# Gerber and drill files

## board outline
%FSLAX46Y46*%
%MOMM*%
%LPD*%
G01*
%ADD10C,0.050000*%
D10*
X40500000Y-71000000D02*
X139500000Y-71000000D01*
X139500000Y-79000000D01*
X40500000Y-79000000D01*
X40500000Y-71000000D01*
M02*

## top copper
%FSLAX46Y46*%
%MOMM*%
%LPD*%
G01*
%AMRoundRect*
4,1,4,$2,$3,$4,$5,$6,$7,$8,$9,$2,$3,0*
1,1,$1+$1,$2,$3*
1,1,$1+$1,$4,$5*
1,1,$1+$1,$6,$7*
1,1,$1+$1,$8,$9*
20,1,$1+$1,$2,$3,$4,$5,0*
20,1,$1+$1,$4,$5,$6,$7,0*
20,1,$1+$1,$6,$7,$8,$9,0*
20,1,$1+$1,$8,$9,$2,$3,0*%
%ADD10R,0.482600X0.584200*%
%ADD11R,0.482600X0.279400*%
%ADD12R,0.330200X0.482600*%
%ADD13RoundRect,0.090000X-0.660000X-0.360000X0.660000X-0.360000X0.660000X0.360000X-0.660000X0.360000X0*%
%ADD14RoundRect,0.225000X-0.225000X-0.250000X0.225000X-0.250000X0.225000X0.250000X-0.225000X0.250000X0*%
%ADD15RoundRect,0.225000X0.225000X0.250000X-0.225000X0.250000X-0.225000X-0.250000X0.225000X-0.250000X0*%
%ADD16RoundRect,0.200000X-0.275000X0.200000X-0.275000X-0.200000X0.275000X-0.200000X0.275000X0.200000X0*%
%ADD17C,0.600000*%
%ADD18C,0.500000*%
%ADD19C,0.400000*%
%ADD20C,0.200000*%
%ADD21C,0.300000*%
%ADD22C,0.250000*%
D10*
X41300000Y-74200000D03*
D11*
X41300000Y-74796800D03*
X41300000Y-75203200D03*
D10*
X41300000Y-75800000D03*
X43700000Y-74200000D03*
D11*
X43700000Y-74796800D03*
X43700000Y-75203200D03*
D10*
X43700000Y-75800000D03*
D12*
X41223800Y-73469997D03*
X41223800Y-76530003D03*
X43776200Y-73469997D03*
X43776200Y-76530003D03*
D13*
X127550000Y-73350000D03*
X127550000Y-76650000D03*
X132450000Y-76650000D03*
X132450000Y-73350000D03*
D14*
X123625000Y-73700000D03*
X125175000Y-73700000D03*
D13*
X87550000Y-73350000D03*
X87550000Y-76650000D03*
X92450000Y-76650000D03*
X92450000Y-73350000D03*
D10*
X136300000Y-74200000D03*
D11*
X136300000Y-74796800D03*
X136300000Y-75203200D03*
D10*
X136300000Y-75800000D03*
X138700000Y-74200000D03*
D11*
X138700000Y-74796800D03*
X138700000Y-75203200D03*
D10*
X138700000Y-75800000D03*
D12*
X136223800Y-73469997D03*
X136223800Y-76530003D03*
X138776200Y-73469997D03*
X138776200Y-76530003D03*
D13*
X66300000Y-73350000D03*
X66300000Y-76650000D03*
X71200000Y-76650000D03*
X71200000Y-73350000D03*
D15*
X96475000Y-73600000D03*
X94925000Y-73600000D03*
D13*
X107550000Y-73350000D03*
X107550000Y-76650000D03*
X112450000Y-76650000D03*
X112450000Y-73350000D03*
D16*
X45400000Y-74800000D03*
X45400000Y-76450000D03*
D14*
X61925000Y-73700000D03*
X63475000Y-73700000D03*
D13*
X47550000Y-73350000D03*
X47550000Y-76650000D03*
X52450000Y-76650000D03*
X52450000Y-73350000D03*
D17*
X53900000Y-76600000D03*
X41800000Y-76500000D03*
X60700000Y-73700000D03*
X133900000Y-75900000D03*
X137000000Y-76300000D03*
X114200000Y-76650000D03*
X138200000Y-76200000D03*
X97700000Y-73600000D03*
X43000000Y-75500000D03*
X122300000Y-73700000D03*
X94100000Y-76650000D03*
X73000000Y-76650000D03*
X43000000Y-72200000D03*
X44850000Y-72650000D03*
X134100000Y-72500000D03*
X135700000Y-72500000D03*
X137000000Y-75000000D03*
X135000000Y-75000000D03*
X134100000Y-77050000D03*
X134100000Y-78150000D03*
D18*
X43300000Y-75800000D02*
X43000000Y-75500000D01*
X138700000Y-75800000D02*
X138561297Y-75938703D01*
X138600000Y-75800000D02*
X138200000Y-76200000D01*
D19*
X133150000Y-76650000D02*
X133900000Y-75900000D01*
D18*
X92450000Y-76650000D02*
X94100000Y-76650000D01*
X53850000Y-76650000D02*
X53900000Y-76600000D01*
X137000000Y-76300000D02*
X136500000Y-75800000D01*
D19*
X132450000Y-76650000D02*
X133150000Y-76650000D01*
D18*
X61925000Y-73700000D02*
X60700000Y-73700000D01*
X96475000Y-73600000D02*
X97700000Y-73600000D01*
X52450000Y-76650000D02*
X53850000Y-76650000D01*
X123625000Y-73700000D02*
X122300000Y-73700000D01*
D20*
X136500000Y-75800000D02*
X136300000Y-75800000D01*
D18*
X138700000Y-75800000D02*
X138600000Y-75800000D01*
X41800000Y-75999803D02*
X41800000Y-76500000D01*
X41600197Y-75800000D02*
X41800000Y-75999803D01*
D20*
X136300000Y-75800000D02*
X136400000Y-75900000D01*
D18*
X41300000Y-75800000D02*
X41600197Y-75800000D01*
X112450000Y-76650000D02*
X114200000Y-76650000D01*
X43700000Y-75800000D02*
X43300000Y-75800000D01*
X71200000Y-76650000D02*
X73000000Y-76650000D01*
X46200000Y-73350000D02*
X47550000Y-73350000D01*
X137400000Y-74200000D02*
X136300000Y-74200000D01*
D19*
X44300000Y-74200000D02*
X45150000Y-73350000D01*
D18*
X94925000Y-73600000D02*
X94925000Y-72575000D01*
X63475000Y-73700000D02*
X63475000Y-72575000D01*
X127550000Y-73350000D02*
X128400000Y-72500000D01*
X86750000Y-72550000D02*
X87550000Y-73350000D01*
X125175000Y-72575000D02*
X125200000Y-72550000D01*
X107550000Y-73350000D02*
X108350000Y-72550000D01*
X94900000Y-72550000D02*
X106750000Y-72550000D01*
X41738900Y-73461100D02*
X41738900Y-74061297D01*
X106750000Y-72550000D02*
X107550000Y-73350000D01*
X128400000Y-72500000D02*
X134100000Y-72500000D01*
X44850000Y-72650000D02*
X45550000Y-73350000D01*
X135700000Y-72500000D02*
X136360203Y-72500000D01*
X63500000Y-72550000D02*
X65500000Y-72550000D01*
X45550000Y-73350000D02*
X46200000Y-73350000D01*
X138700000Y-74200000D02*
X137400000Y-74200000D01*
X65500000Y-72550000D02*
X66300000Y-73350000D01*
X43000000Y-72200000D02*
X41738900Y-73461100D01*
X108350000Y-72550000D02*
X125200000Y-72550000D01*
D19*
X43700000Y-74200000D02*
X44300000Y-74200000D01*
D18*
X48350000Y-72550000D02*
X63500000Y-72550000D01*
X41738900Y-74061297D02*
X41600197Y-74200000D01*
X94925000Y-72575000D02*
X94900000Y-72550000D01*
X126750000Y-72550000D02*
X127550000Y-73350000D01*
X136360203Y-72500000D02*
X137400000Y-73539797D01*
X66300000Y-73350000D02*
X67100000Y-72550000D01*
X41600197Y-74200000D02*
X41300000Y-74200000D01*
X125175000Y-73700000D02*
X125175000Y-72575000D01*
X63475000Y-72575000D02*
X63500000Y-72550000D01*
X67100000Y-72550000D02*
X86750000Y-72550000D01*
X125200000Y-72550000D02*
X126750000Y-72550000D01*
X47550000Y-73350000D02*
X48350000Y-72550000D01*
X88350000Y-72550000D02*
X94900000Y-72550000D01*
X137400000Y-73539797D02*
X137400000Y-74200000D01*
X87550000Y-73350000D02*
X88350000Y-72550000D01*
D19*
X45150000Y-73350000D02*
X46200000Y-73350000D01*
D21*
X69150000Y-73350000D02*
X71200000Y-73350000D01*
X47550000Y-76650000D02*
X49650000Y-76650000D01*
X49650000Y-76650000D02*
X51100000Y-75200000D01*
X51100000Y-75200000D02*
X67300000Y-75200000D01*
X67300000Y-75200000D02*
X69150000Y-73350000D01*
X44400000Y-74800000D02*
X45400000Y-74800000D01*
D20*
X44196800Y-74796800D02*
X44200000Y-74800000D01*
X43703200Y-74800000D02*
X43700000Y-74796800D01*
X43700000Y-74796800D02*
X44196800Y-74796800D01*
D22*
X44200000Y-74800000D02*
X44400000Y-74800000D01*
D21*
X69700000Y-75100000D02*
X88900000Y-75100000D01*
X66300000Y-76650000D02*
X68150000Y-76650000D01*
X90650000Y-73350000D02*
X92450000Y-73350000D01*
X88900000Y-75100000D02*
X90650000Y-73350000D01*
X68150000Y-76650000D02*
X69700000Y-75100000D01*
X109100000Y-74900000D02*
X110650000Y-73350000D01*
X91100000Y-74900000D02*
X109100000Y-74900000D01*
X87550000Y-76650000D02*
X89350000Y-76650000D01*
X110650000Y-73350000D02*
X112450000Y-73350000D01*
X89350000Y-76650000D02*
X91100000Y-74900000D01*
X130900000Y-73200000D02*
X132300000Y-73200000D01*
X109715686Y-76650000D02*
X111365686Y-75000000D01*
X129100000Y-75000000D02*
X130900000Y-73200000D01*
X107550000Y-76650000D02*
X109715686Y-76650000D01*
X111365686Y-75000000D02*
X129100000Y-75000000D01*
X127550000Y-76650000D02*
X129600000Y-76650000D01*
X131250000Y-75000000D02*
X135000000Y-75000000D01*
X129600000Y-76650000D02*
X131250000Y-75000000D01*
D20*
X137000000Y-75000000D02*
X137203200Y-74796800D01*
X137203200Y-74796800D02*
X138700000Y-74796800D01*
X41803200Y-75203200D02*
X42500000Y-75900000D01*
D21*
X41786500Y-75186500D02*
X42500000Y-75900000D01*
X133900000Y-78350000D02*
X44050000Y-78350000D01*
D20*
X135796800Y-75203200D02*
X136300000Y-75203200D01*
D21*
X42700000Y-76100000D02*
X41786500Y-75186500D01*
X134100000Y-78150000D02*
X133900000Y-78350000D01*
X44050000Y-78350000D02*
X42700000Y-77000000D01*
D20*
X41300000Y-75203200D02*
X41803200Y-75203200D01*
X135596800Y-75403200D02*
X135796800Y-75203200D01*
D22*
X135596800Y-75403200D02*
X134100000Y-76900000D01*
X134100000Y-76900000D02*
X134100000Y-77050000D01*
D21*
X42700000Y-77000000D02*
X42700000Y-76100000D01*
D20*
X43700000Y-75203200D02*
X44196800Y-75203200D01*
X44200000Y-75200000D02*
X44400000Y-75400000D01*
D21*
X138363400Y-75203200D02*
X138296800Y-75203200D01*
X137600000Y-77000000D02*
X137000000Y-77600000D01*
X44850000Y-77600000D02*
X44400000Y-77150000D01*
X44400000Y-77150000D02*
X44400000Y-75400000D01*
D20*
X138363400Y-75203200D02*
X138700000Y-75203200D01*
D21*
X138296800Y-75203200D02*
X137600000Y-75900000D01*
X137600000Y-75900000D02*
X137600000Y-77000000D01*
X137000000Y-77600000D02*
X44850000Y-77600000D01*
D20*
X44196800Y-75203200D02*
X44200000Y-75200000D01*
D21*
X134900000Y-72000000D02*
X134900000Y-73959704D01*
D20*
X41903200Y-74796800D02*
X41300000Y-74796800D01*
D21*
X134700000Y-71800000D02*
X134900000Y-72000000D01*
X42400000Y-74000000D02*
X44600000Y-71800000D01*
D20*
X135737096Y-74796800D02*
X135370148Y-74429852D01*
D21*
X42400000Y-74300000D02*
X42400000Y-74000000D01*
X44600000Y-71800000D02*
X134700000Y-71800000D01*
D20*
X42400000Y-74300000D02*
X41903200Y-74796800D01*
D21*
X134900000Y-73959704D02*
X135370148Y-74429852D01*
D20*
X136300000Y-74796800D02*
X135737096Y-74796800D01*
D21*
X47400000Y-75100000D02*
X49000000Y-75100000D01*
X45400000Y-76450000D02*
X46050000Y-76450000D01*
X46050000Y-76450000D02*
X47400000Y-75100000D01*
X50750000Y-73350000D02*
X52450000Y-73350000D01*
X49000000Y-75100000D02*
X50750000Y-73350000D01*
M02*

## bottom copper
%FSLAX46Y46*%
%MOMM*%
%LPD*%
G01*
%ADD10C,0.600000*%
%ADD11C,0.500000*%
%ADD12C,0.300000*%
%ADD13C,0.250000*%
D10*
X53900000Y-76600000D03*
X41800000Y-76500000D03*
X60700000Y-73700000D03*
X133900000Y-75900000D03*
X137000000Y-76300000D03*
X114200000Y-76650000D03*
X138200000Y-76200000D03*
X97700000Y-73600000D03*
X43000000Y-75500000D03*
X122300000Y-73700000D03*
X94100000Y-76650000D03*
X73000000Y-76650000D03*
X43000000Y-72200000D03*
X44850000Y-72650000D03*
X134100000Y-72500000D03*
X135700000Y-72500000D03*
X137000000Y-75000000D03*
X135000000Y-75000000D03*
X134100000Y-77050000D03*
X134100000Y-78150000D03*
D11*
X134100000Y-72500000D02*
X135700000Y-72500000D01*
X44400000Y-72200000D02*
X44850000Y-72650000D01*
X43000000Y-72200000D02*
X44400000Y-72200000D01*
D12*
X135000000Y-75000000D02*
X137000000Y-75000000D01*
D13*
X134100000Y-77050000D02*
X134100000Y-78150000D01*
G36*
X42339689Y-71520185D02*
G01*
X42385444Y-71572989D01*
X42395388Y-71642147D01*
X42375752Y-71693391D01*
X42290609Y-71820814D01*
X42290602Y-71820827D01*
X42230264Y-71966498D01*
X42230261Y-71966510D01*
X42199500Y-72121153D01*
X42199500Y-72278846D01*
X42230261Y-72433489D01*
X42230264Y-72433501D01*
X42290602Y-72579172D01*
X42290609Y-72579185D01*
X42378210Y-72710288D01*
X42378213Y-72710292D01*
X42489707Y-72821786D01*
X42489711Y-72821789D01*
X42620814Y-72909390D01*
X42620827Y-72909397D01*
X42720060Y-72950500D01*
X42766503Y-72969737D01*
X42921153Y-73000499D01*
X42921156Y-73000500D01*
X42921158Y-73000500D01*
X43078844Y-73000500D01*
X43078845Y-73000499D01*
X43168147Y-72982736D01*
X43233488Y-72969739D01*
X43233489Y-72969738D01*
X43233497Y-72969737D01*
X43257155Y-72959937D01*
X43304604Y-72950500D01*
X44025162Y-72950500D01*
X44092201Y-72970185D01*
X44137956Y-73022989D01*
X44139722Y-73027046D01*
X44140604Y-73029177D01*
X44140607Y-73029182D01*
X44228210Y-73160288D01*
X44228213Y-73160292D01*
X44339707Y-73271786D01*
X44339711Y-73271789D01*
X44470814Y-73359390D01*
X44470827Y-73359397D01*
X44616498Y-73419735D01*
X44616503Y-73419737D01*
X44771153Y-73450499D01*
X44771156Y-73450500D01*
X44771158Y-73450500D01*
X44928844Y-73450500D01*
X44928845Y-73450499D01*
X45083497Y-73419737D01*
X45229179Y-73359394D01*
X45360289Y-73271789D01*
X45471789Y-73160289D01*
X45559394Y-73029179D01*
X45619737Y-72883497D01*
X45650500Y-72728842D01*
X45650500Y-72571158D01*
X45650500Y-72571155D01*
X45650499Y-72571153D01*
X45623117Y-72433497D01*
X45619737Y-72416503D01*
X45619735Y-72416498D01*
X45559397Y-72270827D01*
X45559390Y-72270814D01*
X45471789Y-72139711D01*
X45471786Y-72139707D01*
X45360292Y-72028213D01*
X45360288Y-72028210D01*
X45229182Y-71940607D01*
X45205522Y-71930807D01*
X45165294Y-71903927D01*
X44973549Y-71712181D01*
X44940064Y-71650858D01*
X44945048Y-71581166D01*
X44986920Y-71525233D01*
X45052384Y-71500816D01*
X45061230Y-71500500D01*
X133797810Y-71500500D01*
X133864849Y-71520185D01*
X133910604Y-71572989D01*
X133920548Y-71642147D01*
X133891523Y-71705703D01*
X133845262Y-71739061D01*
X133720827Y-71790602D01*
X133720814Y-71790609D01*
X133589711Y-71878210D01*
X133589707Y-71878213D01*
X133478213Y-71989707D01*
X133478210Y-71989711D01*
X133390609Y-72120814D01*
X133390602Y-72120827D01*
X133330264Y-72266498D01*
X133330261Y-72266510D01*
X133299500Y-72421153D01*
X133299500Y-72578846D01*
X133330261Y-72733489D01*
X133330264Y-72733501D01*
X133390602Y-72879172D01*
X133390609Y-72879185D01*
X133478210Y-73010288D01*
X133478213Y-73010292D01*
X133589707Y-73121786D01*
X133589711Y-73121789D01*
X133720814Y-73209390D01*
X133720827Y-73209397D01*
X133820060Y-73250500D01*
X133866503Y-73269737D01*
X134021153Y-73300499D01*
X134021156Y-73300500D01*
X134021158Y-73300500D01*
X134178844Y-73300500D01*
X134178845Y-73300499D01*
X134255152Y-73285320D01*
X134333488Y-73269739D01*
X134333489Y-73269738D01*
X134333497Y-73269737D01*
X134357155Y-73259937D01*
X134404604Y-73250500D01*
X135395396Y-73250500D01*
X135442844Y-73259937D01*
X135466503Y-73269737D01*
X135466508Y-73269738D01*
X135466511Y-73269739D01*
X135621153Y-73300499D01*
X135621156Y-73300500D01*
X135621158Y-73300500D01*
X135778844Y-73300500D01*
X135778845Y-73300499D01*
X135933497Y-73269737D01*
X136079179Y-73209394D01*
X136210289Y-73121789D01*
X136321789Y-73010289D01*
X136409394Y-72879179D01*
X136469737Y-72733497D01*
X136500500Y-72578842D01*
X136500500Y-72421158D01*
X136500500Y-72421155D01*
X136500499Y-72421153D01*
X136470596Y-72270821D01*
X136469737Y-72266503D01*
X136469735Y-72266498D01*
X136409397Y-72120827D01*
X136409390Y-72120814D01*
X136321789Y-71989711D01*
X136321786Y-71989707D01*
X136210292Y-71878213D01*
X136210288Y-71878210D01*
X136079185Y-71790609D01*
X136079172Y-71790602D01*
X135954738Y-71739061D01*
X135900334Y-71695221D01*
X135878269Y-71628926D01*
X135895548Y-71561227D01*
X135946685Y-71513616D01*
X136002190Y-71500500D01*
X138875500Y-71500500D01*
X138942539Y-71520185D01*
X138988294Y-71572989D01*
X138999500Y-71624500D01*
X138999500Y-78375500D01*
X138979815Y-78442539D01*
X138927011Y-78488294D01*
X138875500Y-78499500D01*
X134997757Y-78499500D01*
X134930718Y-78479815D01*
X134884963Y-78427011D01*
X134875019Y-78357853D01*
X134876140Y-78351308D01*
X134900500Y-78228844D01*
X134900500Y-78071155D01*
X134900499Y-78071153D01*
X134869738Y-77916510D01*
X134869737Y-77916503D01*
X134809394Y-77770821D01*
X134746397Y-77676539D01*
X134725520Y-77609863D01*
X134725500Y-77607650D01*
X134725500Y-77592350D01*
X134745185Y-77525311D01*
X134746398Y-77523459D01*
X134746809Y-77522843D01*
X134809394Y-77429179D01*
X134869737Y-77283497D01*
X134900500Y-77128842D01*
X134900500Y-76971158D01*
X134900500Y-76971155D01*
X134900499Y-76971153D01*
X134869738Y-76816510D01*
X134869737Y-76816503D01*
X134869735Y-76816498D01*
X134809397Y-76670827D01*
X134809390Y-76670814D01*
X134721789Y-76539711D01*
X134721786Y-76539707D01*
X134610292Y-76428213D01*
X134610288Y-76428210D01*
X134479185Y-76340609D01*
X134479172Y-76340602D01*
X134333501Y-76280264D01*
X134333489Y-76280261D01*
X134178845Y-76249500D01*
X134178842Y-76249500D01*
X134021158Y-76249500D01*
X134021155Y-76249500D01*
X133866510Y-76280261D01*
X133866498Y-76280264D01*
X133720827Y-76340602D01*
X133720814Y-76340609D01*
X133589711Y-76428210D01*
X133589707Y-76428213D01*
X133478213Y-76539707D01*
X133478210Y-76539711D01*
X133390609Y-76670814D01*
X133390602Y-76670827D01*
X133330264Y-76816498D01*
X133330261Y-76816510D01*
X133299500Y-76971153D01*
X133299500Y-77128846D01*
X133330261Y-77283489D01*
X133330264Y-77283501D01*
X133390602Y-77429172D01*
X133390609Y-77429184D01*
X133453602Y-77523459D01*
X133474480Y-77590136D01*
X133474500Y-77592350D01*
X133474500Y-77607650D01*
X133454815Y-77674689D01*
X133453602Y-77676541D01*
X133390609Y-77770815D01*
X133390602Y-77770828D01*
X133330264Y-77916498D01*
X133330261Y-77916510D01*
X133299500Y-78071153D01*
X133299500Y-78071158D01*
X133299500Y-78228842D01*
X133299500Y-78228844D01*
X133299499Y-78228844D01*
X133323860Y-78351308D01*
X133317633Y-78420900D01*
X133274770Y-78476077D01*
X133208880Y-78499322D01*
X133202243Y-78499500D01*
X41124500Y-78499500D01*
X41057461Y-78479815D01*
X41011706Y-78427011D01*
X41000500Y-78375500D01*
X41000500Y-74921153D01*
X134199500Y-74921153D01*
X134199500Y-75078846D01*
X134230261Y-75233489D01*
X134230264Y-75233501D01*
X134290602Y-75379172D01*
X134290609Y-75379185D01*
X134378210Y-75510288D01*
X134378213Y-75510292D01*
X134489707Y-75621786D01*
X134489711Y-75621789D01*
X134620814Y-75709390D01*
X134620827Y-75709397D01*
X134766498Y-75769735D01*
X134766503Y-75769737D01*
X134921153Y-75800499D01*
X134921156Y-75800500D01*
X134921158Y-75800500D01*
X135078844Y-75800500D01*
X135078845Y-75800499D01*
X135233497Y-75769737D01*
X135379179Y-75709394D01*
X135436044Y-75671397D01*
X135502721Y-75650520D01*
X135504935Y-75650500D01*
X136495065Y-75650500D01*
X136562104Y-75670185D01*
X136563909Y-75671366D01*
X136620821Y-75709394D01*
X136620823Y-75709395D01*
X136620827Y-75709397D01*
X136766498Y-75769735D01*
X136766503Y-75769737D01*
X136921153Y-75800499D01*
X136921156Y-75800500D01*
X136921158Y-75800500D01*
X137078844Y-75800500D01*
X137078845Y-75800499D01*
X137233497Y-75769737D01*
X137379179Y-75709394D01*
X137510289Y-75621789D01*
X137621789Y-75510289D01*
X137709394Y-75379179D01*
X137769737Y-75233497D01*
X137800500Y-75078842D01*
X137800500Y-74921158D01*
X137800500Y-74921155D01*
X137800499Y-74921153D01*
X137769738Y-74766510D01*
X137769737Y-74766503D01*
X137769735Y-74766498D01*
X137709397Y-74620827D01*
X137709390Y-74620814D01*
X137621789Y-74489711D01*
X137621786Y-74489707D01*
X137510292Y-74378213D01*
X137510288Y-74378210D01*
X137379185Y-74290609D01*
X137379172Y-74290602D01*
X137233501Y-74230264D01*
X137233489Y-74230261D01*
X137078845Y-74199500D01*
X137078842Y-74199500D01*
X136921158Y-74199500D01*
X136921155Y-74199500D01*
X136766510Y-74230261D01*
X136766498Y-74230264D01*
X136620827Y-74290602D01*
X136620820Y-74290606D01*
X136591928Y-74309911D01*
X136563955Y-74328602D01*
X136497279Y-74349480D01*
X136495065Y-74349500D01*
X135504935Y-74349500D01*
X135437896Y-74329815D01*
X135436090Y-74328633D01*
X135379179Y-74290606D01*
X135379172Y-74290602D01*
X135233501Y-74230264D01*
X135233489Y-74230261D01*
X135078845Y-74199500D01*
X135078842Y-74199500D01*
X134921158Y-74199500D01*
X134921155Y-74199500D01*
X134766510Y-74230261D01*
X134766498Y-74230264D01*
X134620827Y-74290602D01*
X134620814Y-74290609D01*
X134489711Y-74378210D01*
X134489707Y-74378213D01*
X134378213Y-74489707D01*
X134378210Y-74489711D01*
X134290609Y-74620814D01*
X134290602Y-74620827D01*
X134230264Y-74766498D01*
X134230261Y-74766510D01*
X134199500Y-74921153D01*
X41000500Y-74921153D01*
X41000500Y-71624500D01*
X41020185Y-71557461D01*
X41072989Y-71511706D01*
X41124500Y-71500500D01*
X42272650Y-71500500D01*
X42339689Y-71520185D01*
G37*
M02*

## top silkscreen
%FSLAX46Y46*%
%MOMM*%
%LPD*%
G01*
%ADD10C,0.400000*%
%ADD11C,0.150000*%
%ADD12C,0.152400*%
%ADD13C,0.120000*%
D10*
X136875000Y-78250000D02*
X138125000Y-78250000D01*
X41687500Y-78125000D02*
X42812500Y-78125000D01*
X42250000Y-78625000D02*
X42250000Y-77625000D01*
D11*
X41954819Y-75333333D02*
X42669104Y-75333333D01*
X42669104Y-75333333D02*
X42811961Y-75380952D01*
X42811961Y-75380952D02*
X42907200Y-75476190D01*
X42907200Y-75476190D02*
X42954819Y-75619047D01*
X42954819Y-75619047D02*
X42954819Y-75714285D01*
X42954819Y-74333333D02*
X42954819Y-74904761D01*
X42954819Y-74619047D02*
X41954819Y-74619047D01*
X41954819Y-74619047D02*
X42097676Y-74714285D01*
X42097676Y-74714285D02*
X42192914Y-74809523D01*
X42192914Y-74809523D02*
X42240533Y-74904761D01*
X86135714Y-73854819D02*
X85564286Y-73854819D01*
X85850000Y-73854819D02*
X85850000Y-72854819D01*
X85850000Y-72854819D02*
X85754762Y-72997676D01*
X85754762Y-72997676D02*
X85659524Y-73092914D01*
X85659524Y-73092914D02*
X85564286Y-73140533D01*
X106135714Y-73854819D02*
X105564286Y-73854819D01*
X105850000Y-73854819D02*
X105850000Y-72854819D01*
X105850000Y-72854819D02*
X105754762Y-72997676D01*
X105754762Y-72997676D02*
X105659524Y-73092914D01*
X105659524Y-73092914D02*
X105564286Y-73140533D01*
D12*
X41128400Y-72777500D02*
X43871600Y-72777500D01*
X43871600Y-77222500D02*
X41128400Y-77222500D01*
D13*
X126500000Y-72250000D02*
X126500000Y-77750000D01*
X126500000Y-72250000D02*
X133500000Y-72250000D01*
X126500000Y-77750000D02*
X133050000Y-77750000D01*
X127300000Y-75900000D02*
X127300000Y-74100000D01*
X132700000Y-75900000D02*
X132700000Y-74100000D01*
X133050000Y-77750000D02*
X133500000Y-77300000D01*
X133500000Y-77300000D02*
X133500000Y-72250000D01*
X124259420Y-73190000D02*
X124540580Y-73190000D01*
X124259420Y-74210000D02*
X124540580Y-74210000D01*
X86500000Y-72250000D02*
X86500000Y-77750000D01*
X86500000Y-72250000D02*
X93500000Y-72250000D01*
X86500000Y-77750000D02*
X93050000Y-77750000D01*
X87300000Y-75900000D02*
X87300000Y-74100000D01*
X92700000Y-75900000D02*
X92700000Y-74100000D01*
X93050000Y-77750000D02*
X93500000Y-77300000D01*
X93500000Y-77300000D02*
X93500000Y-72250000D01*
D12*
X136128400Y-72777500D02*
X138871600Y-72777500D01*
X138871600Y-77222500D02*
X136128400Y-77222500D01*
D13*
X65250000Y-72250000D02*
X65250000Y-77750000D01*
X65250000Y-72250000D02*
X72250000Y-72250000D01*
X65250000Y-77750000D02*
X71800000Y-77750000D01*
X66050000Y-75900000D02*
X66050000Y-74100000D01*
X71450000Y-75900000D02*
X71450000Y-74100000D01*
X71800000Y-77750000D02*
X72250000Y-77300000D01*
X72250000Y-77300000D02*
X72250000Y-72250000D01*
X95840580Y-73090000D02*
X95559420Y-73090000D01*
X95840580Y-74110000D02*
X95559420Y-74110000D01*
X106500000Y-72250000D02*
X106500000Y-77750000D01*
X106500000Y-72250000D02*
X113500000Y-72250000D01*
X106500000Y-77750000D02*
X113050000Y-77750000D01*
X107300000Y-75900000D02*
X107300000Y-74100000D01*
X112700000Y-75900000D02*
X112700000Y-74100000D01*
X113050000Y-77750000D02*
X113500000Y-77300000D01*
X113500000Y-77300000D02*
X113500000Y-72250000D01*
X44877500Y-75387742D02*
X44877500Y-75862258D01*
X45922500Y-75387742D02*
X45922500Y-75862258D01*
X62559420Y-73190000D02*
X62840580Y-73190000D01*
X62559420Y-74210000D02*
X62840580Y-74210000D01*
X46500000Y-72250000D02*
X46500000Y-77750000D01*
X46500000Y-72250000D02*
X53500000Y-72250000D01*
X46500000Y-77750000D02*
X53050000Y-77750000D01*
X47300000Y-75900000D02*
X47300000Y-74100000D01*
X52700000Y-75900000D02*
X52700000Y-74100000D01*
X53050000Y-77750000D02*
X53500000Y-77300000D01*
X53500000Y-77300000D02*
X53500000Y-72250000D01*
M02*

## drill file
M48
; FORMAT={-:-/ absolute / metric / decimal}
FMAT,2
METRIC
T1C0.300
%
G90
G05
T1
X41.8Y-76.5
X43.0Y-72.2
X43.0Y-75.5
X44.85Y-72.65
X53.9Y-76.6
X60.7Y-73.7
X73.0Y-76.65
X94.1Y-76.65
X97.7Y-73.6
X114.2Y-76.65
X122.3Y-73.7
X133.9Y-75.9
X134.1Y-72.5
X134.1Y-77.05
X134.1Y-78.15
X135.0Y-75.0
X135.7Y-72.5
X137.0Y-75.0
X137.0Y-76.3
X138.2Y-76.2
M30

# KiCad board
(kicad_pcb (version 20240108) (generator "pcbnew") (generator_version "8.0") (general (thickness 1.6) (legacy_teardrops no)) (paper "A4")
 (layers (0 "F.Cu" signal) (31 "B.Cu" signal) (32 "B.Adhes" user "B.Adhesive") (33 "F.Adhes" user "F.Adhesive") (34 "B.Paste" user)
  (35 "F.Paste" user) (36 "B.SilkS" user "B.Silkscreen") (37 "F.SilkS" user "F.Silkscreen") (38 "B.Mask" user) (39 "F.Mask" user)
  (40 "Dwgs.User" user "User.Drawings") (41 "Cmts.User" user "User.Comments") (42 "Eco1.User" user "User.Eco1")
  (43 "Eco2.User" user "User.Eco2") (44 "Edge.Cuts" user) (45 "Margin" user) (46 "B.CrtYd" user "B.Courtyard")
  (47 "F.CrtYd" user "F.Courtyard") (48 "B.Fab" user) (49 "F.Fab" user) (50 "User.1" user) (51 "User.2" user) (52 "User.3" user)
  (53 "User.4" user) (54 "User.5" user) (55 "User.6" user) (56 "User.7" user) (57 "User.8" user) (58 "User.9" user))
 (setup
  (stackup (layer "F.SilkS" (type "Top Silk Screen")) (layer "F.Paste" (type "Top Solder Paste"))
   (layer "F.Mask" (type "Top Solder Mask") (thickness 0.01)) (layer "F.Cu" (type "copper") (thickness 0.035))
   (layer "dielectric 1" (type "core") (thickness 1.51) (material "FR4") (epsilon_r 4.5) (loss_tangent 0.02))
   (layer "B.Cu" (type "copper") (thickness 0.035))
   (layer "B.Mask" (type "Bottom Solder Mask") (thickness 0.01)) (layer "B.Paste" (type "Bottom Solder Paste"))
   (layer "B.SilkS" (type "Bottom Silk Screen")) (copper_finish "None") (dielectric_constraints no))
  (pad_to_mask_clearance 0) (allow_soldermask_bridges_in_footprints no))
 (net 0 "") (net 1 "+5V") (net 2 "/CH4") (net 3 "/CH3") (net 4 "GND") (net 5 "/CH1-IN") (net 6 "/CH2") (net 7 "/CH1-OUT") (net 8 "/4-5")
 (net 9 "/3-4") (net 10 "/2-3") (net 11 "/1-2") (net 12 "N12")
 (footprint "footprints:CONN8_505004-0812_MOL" (layer "F.Cu") (at 42.5 75 90)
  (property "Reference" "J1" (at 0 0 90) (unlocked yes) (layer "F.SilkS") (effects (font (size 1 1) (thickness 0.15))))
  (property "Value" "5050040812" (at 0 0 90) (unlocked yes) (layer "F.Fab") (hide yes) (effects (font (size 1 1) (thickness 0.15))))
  (fp_line (start 2.2225 -1.3716) (end 2.2225 1.3716) (stroke (width 0.1524) (type solid)) (layer "F.SilkS"))
  (fp_line (start -2.2225 1.3716) (end -2.2225 -1.3716) (stroke (width 0.1524) (type solid)) (layer "F.SilkS"))
  (pad "1" smd rect (at 0.8 -1.2 90) (size 0.5842 0.4826) (layers "F.Cu" "F.Paste" "F.Mask") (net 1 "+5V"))
  (pad "2" smd rect (at 0.2032 -1.2 90) (size 0.2794 0.4826) (layers "F.Cu" "F.Paste" "F.Mask") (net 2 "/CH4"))
  (pad "3" smd rect (at -0.2032 -1.2 90) (size 0.2794 0.4826) (layers "F.Cu" "F.Paste" "F.Mask") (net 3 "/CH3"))
  (pad "4" smd rect (at -0.8 -1.2 90) (size 0.5842 0.4826) (layers "F.Cu" "F.Paste" "F.Mask") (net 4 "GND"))
  (pad "5" smd rect (at 0.8 1.2 90) (size 0.5842 0.4826) (layers "F.Cu" "F.Paste" "F.Mask") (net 1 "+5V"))
  (pad "6" smd rect (at 0.2032 1.2 90) (size 0.2794 0.4826) (layers "F.Cu" "F.Paste" "F.Mask") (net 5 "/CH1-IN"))
  (pad "7" smd rect (at -0.2032 1.2 90) (size 0.2794 0.4826) (layers "F.Cu" "F.Paste" "F.Mask") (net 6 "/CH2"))
  (pad "8" smd rect (at -0.8 1.2 90) (size 0.5842 0.4826) (layers "F.Cu" "F.Paste" "F.Mask") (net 4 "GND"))
  (pad "9" smd rect (at 1.530003 -1.2762 90) (size 0.4826 0.3302) (layers "F.Cu" "F.Paste" "F.Mask"))
  (pad "10" smd rect (at -1.530003 -1.2762 90) (size 0.4826 0.3302) (layers "F.Cu" "F.Paste" "F.Mask"))
  (pad "11" smd rect (at 1.530003 1.2762 90) (size 0.4826 0.3302) (layers "F.Cu" "F.Paste" "F.Mask"))
  (pad "12" smd rect (at -1.530003 1.2762 90) (size 0.4826 0.3302) (layers "F.Cu" "F.Paste" "F.Mask")))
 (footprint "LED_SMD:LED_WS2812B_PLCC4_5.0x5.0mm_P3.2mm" (layer "F.Cu") (at 130 75)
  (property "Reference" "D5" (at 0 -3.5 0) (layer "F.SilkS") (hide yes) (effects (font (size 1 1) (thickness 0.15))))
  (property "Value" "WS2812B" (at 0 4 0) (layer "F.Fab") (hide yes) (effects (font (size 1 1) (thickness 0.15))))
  (fp_line (start -3.5 -2.75) (end -3.5 2.75) (stroke (width 0.12) (type default)) (layer "F.SilkS"))
  (fp_line (start -3.5 -2.75) (end 3.5 -2.75) (stroke (width 0.12) (type solid)) (layer "F.SilkS"))
  (fp_line (start -3.5 2.75) (end 3.05 2.75) (stroke (width 0.12) (type solid)) (layer "F.SilkS"))
  (fp_line (start -2.7 0.9) (end -2.7 -0.9) (stroke (width 0.12) (type default)) (layer "F.SilkS"))
  (fp_line (start 2.7 0.9) (end 2.7 -0.9) (stroke (width 0.12) (type default)) (layer "F.SilkS"))
  (fp_line (start 3.05 2.75) (end 3.5 2.3) (stroke (width 0.12) (type default)) (layer "F.SilkS"))
  (fp_line (start 3.5 2.3) (end 3.5 -2.75) (stroke (width 0.12) (type default)) (layer "F.SilkS"))
  (pad "1" smd roundrect (at -2.45 -1.65) (size 1.5 0.9) (layers "F.Cu" "F.Paste" "F.Mask") (roundrect_rratio 0.1) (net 1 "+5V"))
  (pad "2" smd roundrect (at -2.45 1.65) (size 1.5 0.9) (layers "F.Cu" "F.Paste" "F.Mask") (roundrect_rratio 0.1) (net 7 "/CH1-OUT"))
  (pad "3" smd roundrect (at 2.45 1.65) (size 1.5 0.9) (layers "F.Cu" "F.Paste" "F.Mask") (roundrect_rratio 0.1) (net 4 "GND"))
  (pad "4" smd roundrect (at 2.45 -1.65) (size 1.5 0.9) (layers "F.Cu" "F.Paste" "F.Mask") (roundrect_rratio 0.1) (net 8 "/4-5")))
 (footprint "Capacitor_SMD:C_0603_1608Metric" (layer "F.Cu") (at 124.4 73.7)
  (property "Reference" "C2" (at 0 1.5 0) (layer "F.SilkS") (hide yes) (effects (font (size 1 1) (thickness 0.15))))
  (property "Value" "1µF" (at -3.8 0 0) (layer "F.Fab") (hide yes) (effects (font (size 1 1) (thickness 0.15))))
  (fp_line (start -0.14058 -0.51) (end 0.14058 -0.51) (stroke (width 0.12) (type solid)) (layer "F.SilkS"))
  (fp_line (start -0.14058 0.51) (end 0.14058 0.51) (stroke (width 0.12) (type solid)) (layer "F.SilkS"))
  (pad "1" smd roundrect (at -0.775 0) (size 0.9 0.95) (layers "F.Cu" "F.Paste" "F.Mask") (roundrect_rratio 0.25) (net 4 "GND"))
  (pad "2" smd roundrect (at 0.775 0) (size 0.9 0.95) (layers "F.Cu" "F.Paste" "F.Mask") (roundrect_rratio 0.25) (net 1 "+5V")))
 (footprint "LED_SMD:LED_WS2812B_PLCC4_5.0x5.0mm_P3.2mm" (layer "F.Cu") (at 90 75)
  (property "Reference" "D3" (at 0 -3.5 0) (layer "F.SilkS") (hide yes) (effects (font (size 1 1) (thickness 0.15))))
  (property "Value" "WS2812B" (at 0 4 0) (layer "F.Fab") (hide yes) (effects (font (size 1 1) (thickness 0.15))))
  (fp_line (start -3.5 -2.75) (end -3.5 2.75) (stroke (width 0.12) (type default)) (layer "F.SilkS"))
  (fp_line (start -3.5 -2.75) (end 3.5 -2.75) (stroke (width 0.12) (type solid)) (layer "F.SilkS"))
  (fp_line (start -3.5 2.75) (end 3.05 2.75) (stroke (width 0.12) (type solid)) (layer "F.SilkS"))
  (fp_line (start -2.7 0.9) (end -2.7 -0.9) (stroke (width 0.12) (type default)) (layer "F.SilkS"))
  (fp_line (start 2.7 0.9) (end 2.7 -0.9) (stroke (width 0.12) (type default)) (layer "F.SilkS"))
  (fp_line (start 3.05 2.75) (end 3.5 2.3) (stroke (width 0.12) (type default)) (layer "F.SilkS"))
  (fp_line (start 3.5 2.3) (end 3.5 -2.75) (stroke (width 0.12) (type default)) (layer "F.SilkS"))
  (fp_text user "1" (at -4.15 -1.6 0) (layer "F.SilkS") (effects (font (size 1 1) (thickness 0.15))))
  (pad "1" smd roundrect (at -2.45 -1.65) (size 1.5 0.9) (layers "F.Cu" "F.Paste" "F.Mask") (roundrect_rratio 0.1) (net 1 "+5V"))
  (pad "2" smd roundrect (at -2.45 1.65) (size 1.5 0.9) (layers "F.Cu" "F.Paste" "F.Mask") (roundrect_rratio 0.1) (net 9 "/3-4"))
  (pad "3" smd roundrect (at 2.45 1.65) (size 1.5 0.9) (layers "F.Cu" "F.Paste" "F.Mask") (roundrect_rratio 0.1) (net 4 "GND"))
  (pad "4" smd roundrect (at 2.45 -1.65) (size 1.5 0.9) (layers "F.Cu" "F.Paste" "F.Mask") (roundrect_rratio 0.1) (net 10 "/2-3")))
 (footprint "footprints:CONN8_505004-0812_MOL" (layer "F.Cu") (at 137.5 75 90)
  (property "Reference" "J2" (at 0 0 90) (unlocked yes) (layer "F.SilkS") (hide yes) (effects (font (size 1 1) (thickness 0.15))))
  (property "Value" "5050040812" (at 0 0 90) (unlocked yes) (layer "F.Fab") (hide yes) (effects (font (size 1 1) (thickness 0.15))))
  (fp_line (start 2.2225 -1.3716) (end 2.2225 1.3716) (stroke (width 0.1524) (type solid)) (layer "F.SilkS"))
  (fp_line (start -2.2225 1.3716) (end -2.2225 -1.3716) (stroke (width 0.1524) (type solid)) (layer "F.SilkS"))
  (pad "1" smd rect (at 0.8 -1.2 90) (size 0.5842 0.4826) (layers "F.Cu" "F.Paste" "F.Mask") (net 1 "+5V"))
  (pad "2" smd rect (at 0.2032 -1.2 90) (size 0.2794 0.4826) (layers "F.Cu" "F.Paste" "F.Mask") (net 2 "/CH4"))
  (pad "3" smd rect (at -0.2032 -1.2 90) (size 0.2794 0.4826) (layers "F.Cu" "F.Paste" "F.Mask") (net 3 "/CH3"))
  (pad "4" smd rect (at -0.8 -1.2 90) (size 0.5842 0.4826) (layers "F.Cu" "F.Paste" "F.Mask") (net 4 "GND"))
  (pad "5" smd rect (at 0.8 1.2 90) (size 0.5842 0.4826) (layers "F.Cu" "F.Paste" "F.Mask") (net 1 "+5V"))
  (pad "6" smd rect (at 0.2032 1.2 90) (size 0.2794 0.4826) (layers "F.Cu" "F.Paste" "F.Mask") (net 7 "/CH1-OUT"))
  (pad "7" smd rect (at -0.2032 1.2 90) (size 0.2794 0.4826) (layers "F.Cu" "F.Paste" "F.Mask") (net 6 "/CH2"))
  (pad "8" smd rect (at -0.8 1.2 90) (size 0.5842 0.4826) (layers "F.Cu" "F.Paste" "F.Mask") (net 4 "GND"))
  (pad "9" smd rect (at 1.530003 -1.2762 90) (size 0.4826 0.3302) (layers "F.Cu" "F.Paste" "F.Mask"))
  (pad "10" smd rect (at -1.530003 -1.2762 90) (size 0.4826 0.3302) (layers "F.Cu" "F.Paste" "F.Mask"))
  (pad "11" smd rect (at 1.530003 1.2762 90) (size 0.4826 0.3302) (layers "F.Cu" "F.Paste" "F.Mask"))
  (pad "12" smd rect (at -1.530003 1.2762 90) (size 0.4826 0.3302) (layers "F.Cu" "F.Paste" "F.Mask")))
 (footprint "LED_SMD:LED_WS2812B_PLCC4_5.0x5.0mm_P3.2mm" (layer "F.Cu") (at 68.75 75)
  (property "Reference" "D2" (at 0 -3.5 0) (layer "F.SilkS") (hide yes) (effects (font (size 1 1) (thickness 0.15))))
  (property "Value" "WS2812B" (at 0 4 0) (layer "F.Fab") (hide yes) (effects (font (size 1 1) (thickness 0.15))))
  (fp_line (start -3.5 -2.75) (end -3.5 2.75) (stroke (width 0.12) (type default)) (layer "F.SilkS"))
  (fp_line (start -3.5 -2.75) (end 3.5 -2.75) (stroke (width 0.12) (type solid)) (layer "F.SilkS"))
  (fp_line (start -3.5 2.75) (end 3.05 2.75) (stroke (width 0.12) (type solid)) (layer "F.SilkS"))
  (fp_line (start -2.7 0.9) (end -2.7 -0.9) (stroke (width 0.12) (type default)) (layer "F.SilkS"))
  (fp_line (start 2.7 0.9) (end 2.7 -0.9) (stroke (width 0.12) (type default)) (layer "F.SilkS"))
  (fp_line (start 3.05 2.75) (end 3.5 2.3) (stroke (width 0.12) (type default)) (layer "F.SilkS"))
  (fp_line (start 3.5 2.3) (end 3.5 -2.75) (stroke (width 0.12) (type default)) (layer "F.SilkS"))
  (pad "1" smd roundrect (at -2.45 -1.65) (size 1.5 0.9) (layers "F.Cu" "F.Paste" "F.Mask") (roundrect_rratio 0.1) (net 1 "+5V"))
  (pad "2" smd roundrect (at -2.45 1.65) (size 1.5 0.9) (layers "F.Cu" "F.Paste" "F.Mask") (roundrect_rratio 0.1) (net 10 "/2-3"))
  (pad "3" smd roundrect (at 2.45 1.65) (size 1.5 0.9) (layers "F.Cu" "F.Paste" "F.Mask") (roundrect_rratio 0.1) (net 4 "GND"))
  (pad "4" smd roundrect (at 2.45 -1.65) (size 1.5 0.9) (layers "F.Cu" "F.Paste" "F.Mask") (roundrect_rratio 0.1) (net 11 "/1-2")))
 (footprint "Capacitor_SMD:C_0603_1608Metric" (layer "F.Cu") (at 95.7 73.6 180)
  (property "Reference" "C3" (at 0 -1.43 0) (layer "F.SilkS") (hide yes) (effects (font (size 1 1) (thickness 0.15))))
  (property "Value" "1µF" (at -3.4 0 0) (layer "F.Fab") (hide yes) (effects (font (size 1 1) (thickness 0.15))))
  (fp_line (start -0.14058 0.51) (end 0.14058 0.51) (stroke (width 0.12) (type solid)) (layer "F.SilkS"))
  (fp_line (start -0.14058 -0.51) (end 0.14058 -0.51) (stroke (width 0.12) (type solid)) (layer "F.SilkS"))
  (pad "1" smd roundrect (at -0.775 0 180) (size 0.9 0.95) (layers "F.Cu" "F.Paste" "F.Mask") (roundrect_rratio 0.25) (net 4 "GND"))
  (pad "2" smd roundrect (at 0.775 0 180) (size 0.9 0.95) (layers "F.Cu" "F.Paste" "F.Mask") (roundrect_rratio 0.25) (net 1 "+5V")))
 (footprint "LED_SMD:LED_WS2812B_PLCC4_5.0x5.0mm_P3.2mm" (layer "F.Cu") (at 110 75)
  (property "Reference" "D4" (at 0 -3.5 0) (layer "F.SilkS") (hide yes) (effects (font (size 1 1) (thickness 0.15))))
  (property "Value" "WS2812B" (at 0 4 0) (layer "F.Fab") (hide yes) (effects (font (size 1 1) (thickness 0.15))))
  (fp_line (start -3.5 -2.75) (end -3.5 2.75) (stroke (width 0.12) (type default)) (layer "F.SilkS"))
  (fp_line (start -3.5 -2.75) (end 3.5 -2.75) (stroke (width 0.12) (type solid)) (layer "F.SilkS"))
  (fp_line (start -3.5 2.75) (end 3.05 2.75) (stroke (width 0.12) (type solid)) (layer "F.SilkS"))
  (fp_line (start -2.7 0.9) (end -2.7 -0.9) (stroke (width 0.12) (type default)) (layer "F.SilkS"))
  (fp_line (start 2.7 0.9) (end 2.7 -0.9) (stroke (width 0.12) (type default)) (layer "F.SilkS"))
  (fp_line (start 3.05 2.75) (end 3.5 2.3) (stroke (width 0.12) (type default)) (layer "F.SilkS"))
  (fp_line (start 3.5 2.3) (end 3.5 -2.75) (stroke (width 0.12) (type default)) (layer "F.SilkS"))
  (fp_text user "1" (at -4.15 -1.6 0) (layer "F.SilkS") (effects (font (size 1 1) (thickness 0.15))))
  (pad "1" smd roundrect (at -2.45 -1.65) (size 1.5 0.9) (layers "F.Cu" "F.Paste" "F.Mask") (roundrect_rratio 0.1) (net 1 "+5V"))
  (pad "2" smd roundrect (at -2.45 1.65) (size 1.5 0.9) (layers "F.Cu" "F.Paste" "F.Mask") (roundrect_rratio 0.1) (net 8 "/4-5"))
  (pad "3" smd roundrect (at 2.45 1.65) (size 1.5 0.9) (layers "F.Cu" "F.Paste" "F.Mask") (roundrect_rratio 0.1) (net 4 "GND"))
  (pad "4" smd roundrect (at 2.45 -1.65) (size 1.5 0.9) (layers "F.Cu" "F.Paste" "F.Mask") (roundrect_rratio 0.1) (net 9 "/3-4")))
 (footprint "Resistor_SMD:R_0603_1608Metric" (layer "F.Cu") (at 45.4 75.625 -90)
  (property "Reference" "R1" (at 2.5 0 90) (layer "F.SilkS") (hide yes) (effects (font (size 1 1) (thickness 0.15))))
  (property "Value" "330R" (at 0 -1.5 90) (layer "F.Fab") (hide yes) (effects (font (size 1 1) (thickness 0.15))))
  (fp_line (start -0.237258 0.5225) (end 0.237258 0.5225) (stroke (width 0.12) (type solid)) (layer "F.SilkS"))
  (fp_line (start -0.237258 -0.5225) (end 0.237258 -0.5225) (stroke (width 0.12) (type solid)) (layer "F.SilkS"))
  (pad "1" smd roundrect (at -0.825 0 270) (size 0.8 0.95) (layers "F.Cu" "F.Paste" "F.Mask") (roundrect_rratio 0.25) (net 5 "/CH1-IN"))
  (pad "2" smd roundrect (at 0.825 0 270) (size 0.8 0.95) (layers "F.Cu" "F.Paste" "F.Mask") (roundrect_rratio 0.25) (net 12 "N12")))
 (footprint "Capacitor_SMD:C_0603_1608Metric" (layer "F.Cu") (at 62.7 73.7)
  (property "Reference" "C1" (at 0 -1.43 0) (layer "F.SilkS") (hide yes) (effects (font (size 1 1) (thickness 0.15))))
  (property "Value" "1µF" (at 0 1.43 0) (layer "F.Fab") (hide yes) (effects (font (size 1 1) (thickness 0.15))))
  (fp_line (start -0.14058 -0.51) (end 0.14058 -0.51) (stroke (width 0.12) (type solid)) (layer "F.SilkS"))
  (fp_line (start -0.14058 0.51) (end 0.14058 0.51) (stroke (width 0.12) (type solid)) (layer "F.SilkS"))
  (pad "1" smd roundrect (at -0.775 0) (size 0.9 0.95) (layers "F.Cu" "F.Paste" "F.Mask") (roundrect_rratio 0.25) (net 4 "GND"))
  (pad "2" smd roundrect (at 0.775 0) (size 0.9 0.95) (layers "F.Cu" "F.Paste" "F.Mask") (roundrect_rratio 0.25) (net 1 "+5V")))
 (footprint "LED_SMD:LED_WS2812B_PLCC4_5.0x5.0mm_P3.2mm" (layer "F.Cu") (at 50 75)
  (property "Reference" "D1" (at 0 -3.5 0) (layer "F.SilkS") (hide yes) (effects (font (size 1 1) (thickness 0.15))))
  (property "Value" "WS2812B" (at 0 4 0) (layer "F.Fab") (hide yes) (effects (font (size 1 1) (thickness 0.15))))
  (fp_line (start -3.5 -2.75) (end -3.5 2.75) (stroke (width 0.12) (type default)) (layer "F.SilkS"))
  (fp_line (start -3.5 -2.75) (end 3.5 -2.75) (stroke (width 0.12) (type solid)) (layer "F.SilkS"))
  (fp_line (start -3.5 2.75) (end 3.05 2.75) (stroke (width 0.12) (type solid)) (layer "F.SilkS"))
  (fp_line (start -2.7 0.9) (end -2.7 -0.9) (stroke (width 0.12) (type default)) (layer "F.SilkS"))
  (fp_line (start 2.7 0.9) (end 2.7 -0.9) (stroke (width 0.12) (type default)) (layer "F.SilkS"))
  (fp_line (start 3.05 2.75) (end 3.5 2.3) (stroke (width 0.12) (type default)) (layer "F.SilkS"))
  (fp_line (start 3.5 2.3) (end 3.5 -2.75) (stroke (width 0.12) (type default)) (layer "F.SilkS"))
  (pad "1" smd roundrect (at -2.45 -1.65) (size 1.5 0.9) (layers "F.Cu" "F.Paste" "F.Mask") (roundrect_rratio 0.1) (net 1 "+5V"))
  (pad "2" smd roundrect (at -2.45 1.65) (size 1.5 0.9) (layers "F.Cu" "F.Paste" "F.Mask") (roundrect_rratio 0.1) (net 11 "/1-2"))
  (pad "3" smd roundrect (at 2.45 1.65) (size 1.5 0.9) (layers "F.Cu" "F.Paste" "F.Mask") (roundrect_rratio 0.1) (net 4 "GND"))
  (pad "4" smd roundrect (at 2.45 -1.65) (size 1.5 0.9) (layers "F.Cu" "F.Paste" "F.Mask") (roundrect_rratio 0.1) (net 12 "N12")))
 (gr_line (start 136.875 78.25) (end 138.125 78.25) (stroke (width 0.4) (type default)) (layer "F.SilkS"))
 (gr_line (start 41.6875 78.125) (end 42.8125 78.125) (stroke (width 0.4) (type default)) (layer "F.SilkS"))
 (gr_line (start 42.25 78.625) (end 42.25 77.625) (stroke (width 0.4) (type default)) (layer "F.SilkS"))
 (gr_rect (start 40.5 71) (end 139.5 79) (stroke (width 0.05) (type default)) (fill none) (layer "Edge.Cuts"))
 (segment (start 43.3 75.8) (end 43 75.5) (width 0.5) (layer "F.Cu") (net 4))
 (segment (start 138.7 75.8) (end 138.561297 75.938703) (width 0.5) (layer "F.Cu") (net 4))
 (segment (start 138.6 75.8) (end 138.2 76.2) (width 0.5) (layer "F.Cu") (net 4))
 (segment (start 133.15 76.65) (end 133.9 75.9) (width 0.4) (layer "F.Cu") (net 4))
 (segment (start 92.45 76.65) (end 94.1 76.65) (width 0.5) (layer "F.Cu") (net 4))
 (segment (start 53.85 76.65) (end 53.9 76.6) (width 0.5) (layer "F.Cu") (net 4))
 (segment (start 137 76.3) (end 136.5 75.8) (width 0.5) (layer "F.Cu") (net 4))
 (segment (start 132.45 76.65) (end 133.15 76.65) (width 0.4) (layer "F.Cu") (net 4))
 (segment (start 61.925 73.7) (end 60.7 73.7) (width 0.5) (layer "F.Cu") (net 4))
 (segment (start 96.475 73.6) (end 97.7 73.6) (width 0.5) (layer "F.Cu") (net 4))
 (segment (start 52.45 76.65) (end 53.85 76.65) (width 0.5) (layer "F.Cu") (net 4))
 (segment (start 123.625 73.7) (end 122.3 73.7) (width 0.5) (layer "F.Cu") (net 4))
 (segment (start 136.5 75.8) (end 136.3 75.8) (width 0.2) (layer "F.Cu") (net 4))
 (segment (start 138.7 75.8) (end 138.6 75.8) (width 0.5) (layer "F.Cu") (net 4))
 (segment (start 41.8 75.999803) (end 41.8 76.5) (width 0.5) (layer "F.Cu") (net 4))
 (segment (start 41.600197 75.8) (end 41.8 75.999803) (width 0.5) (layer "F.Cu") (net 4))
 (segment (start 136.3 75.8) (end 136.4 75.9) (width 0.2) (layer "F.Cu") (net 4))
 (segment (start 41.3 75.8) (end 41.600197 75.8) (width 0.5) (layer "F.Cu") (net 4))
 (segment (start 112.45 76.65) (end 114.2 76.65) (width 0.5) (layer "F.Cu") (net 4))
 (segment (start 43.7 75.8) (end 43.3 75.8) (width 0.5) (layer "F.Cu") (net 4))
 (segment (start 71.2 76.65) (end 73 76.65) (width 0.5) (layer "F.Cu") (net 4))
 (via (at 53.9 76.6) (size 0.6) (drill 0.3) (layers "F.Cu" "B.Cu") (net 4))
 (via (at 41.8 76.5) (size 0.6) (drill 0.3) (layers "F.Cu" "B.Cu") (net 4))
 (via (at 60.7 73.7) (size 0.6) (drill 0.3) (layers "F.Cu" "B.Cu") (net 4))
 (via (at 133.9 75.9) (size 0.6) (drill 0.3) (layers "F.Cu" "B.Cu") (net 4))
 (via (at 137 76.3) (size 0.6) (drill 0.3) (layers "F.Cu" "B.Cu") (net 4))
 (via (at 114.2 76.65) (size 0.6) (drill 0.3) (layers "F.Cu" "B.Cu") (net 4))
 (via (at 138.2 76.2) (size 0.6) (drill 0.3) (layers "F.Cu" "B.Cu") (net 4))
 (via (at 97.7 73.6) (size 0.6) (drill 0.3) (layers "F.Cu" "B.Cu") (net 4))
 (via (at 43 75.5) (size 0.6) (drill 0.3) (layers "F.Cu" "B.Cu") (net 4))
 (via (at 122.3 73.7) (size 0.6) (drill 0.3) (layers "F.Cu" "B.Cu") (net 4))
 (via (at 94.1 76.65) (size 0.6) (drill 0.3) (layers "F.Cu" "B.Cu") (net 4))
 (via (at 73 76.65) (size 0.6) (drill 0.3) (layers "F.Cu" "B.Cu") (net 4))
 (segment (start 46.2 73.35) (end 47.55 73.35) (width 0.5) (layer "F.Cu") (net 1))
 (segment (start 137.4 74.2) (end 136.3 74.2) (width 0.5) (layer "F.Cu") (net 1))
 (segment (start 44.3 74.2) (end 45.15 73.35) (width 0.4) (layer "F.Cu") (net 1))
 (segment (start 94.925 73.6) (end 94.925 72.575) (width 0.5) (layer "F.Cu") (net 1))
 (segment (start 63.475 73.7) (end 63.475 72.575) (width 0.5) (layer "F.Cu") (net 1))
 (segment (start 127.55 73.35) (end 128.4 72.5) (width 0.5) (layer "F.Cu") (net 1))
 (segment (start 86.75 72.55) (end 87.55 73.35) (width 0.5) (layer "F.Cu") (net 1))
 (segment (start 125.175 72.575) (end 125.2 72.55) (width 0.5) (layer "F.Cu") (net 1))
 (segment (start 107.55 73.35) (end 108.35 72.55) (width 0.5) (layer "F.Cu") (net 1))
 (segment (start 94.9 72.55) (end 106.75 72.55) (width 0.5) (layer "F.Cu") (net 1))
 (segment (start 41.7389 73.4611) (end 41.7389 74.061297) (width 0.5) (layer "F.Cu") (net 1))
 (segment (start 106.75 72.55) (end 107.55 73.35) (width 0.5) (layer "F.Cu") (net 1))
 (segment (start 128.4 72.5) (end 134.1 72.5) (width 0.5) (layer "F.Cu") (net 1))
 (segment (start 44.85 72.65) (end 45.55 73.35) (width 0.5) (layer "F.Cu") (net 1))
 (segment (start 135.7 72.5) (end 136.360203 72.5) (width 0.5) (layer "F.Cu") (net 1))
 (segment (start 63.5 72.55) (end 65.5 72.55) (width 0.5) (layer "F.Cu") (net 1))
 (segment (start 45.55 73.35) (end 46.2 73.35) (width 0.5) (layer "F.Cu") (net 1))
 (segment (start 138.7 74.2) (end 137.4 74.2) (width 0.5) (layer "F.Cu") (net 1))
 (segment (start 65.5 72.55) (end 66.3 73.35) (width 0.5) (layer "F.Cu") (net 1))
 (segment (start 43 72.2) (end 41.7389 73.4611) (width 0.5) (layer "F.Cu") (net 1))
 (segment (start 108.35 72.55) (end 125.2 72.55) (width 0.5) (layer "F.Cu") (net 1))
 (segment (start 43.7 74.2) (end 44.3 74.2) (width 0.4) (layer "F.Cu") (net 1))
 (segment (start 48.35 72.55) (end 63.5 72.55) (width 0.5) (layer "F.Cu") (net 1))
 (segment (start 41.7389 74.061297) (end 41.600197 74.2) (width 0.5) (layer "F.Cu") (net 1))
 (segment (start 94.925 72.575) (end 94.9 72.55) (width 0.5) (layer "F.Cu") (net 1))
 (segment (start 126.75 72.55) (end 127.55 73.35) (width 0.5) (layer "F.Cu") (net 1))
 (segment (start 136.360203 72.5) (end 137.4 73.539797) (width 0.5) (layer "F.Cu") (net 1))
 (segment (start 66.3 73.35) (end 67.1 72.55) (width 0.5) (layer "F.Cu") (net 1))
 (segment (start 41.600197 74.2) (end 41.3 74.2) (width 0.5) (layer "F.Cu") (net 1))
 (segment (start 125.175 73.7) (end 125.175 72.575) (width 0.5) (layer "F.Cu") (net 1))
 (segment (start 63.475 72.575) (end 63.5 72.55) (width 0.5) (layer "F.Cu") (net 1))
 (segment (start 67.1 72.55) (end 86.75 72.55) (width 0.5) (layer "F.Cu") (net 1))
 (segment (start 125.2 72.55) (end 126.75 72.55) (width 0.5) (layer "F.Cu") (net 1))
 (segment (start 47.55 73.35) (end 48.35 72.55) (width 0.5) (layer "F.Cu") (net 1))
 (segment (start 88.35 72.55) (end 94.9 72.55) (width 0.5) (layer "F.Cu") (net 1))
 (segment (start 137.4 73.539797) (end 137.4 74.2) (width 0.5) (layer "F.Cu") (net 1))
 (segment (start 87.55 73.35) (end 88.35 72.55) (width 0.5) (layer "F.Cu") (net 1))
 (segment (start 45.15 73.35) (end 46.2 73.35) (width 0.4) (layer "F.Cu") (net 1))
 (via (at 43 72.2) (size 0.6) (drill 0.3) (layers "F.Cu" "B.Cu") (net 1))
 (via (at 44.85 72.65) (size 0.6) (drill 0.3) (layers "F.Cu" "B.Cu") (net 1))
 (via (at 134.1 72.5) (size 0.6) (drill 0.3) (layers "F.Cu" "B.Cu") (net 1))
 (via (at 135.7 72.5) (size 0.6) (drill 0.3) (layers "F.Cu" "B.Cu") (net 1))
 (segment (start 134.1 72.5) (end 135.7 72.5) (width 0.5) (layer "B.Cu") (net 1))
 (segment (start 44.4 72.2) (end 44.85 72.65) (width 0.5) (layer "B.Cu") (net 1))
 (segment (start 43 72.2) (end 44.4 72.2) (width 0.5) (layer "B.Cu") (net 1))
 (segment (start 69.15 73.35) (end 71.2 73.35) (width 0.3) (layer "F.Cu") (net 11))
 (segment (start 47.55 76.65) (end 49.65 76.65) (width 0.3) (layer "F.Cu") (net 11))
 (segment (start 49.65 76.65) (end 51.1 75.2) (width 0.3) (layer "F.Cu") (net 11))
 (segment (start 51.1 75.2) (end 67.3 75.2) (width 0.3) (layer "F.Cu") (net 11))
 (segment (start 67.3 75.2) (end 69.15 73.35) (width 0.3) (layer "F.Cu") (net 11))
 (segment (start 44.4 74.8) (end 45.4 74.8) (width 0.3) (layer "F.Cu") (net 5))
 (segment (start 44.1968 74.7968) (end 44.2 74.8) (width 0.2) (layer "F.Cu") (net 5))
 (segment (start 43.7032 74.8) (end 43.7 74.7968) (width 0.2) (layer "F.Cu") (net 5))
 (segment (start 43.7 74.7968) (end 44.1968 74.7968) (width 0.2) (layer "F.Cu") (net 5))
 (segment (start 44.2 74.8) (end 44.4 74.8) (width 0.25) (layer "F.Cu") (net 5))
 (segment (start 69.7 75.1) (end 88.9 75.1) (width 0.3) (layer "F.Cu") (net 10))
 (segment (start 66.3 76.65) (end 68.15 76.65) (width 0.3) (layer "F.Cu") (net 10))
 (segment (start 90.65 73.35) (end 92.45 73.35) (width 0.3) (layer "F.Cu") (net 10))
 (segment (start 88.9 75.1) (end 90.65 73.35) (width 0.3) (layer "F.Cu") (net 10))
 (segment (start 68.15 76.65) (end 69.7 75.1) (width 0.3) (layer "F.Cu") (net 10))
 (segment (start 109.1 74.9) (end 110.65 73.35) (width 0.3) (layer "F.Cu") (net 9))
 (segment (start 91.1 74.9) (end 109.1 74.9) (width 0.3) (layer "F.Cu") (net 9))
 (segment (start 87.55 76.65) (end 89.35 76.65) (width 0.3) (layer "F.Cu") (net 9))
 (segment (start 110.65 73.35) (end 112.45 73.35) (width 0.3) (layer "F.Cu") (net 9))
 (segment (start 89.35 76.65) (end 91.1 74.9) (width 0.3) (layer "F.Cu") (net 9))
 (segment (start 130.9 73.2) (end 132.3 73.2) (width 0.3) (layer "F.Cu") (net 8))
 (segment (start 109.715686 76.65) (end 111.365686 75) (width 0.3) (layer "F.Cu") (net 8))
 (segment (start 129.1 75) (end 130.9 73.2) (width 0.3) (layer "F.Cu") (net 8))
 (segment (start 107.55 76.65) (end 109.715686 76.65) (width 0.3) (layer "F.Cu") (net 8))
 (segment (start 111.365686 75) (end 129.1 75) (width 0.3) (layer "F.Cu") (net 8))
 (segment (start 127.55 76.65) (end 129.6 76.65) (width 0.3) (layer "F.Cu") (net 7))
 (segment (start 131.25 75) (end 135 75) (width 0.3) (layer "F.Cu") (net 7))
 (segment (start 129.6 76.65) (end 131.25 75) (width 0.3) (layer "F.Cu") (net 7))
 (segment (start 137 75) (end 137.2032 74.7968) (width 0.2) (layer "F.Cu") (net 7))
 (segment (start 137.2032 74.7968) (end 138.7 74.7968) (width 0.2) (layer "F.Cu") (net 7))
 (via (at 137 75) (size 0.6) (drill 0.3) (layers "F.Cu" "B.Cu") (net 7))
 (via (at 135 75) (size 0.6) (drill 0.3) (layers "F.Cu" "B.Cu") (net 7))
 (segment (start 135 75) (end 137 75) (width 0.3) (layer "B.Cu") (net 7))
 (segment (start 41.8032 75.2032) (end 42.5 75.9) (width 0.2) (layer "F.Cu") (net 3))
 (segment (start 41.7865 75.1865) (end 42.5 75.9) (width 0.3) (layer "F.Cu") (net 3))
 (segment (start 133.9 78.35) (end 44.05 78.35) (width 0.3) (layer "F.Cu") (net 3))
 (segment (start 135.7968 75.2032) (end 136.3 75.2032) (width 0.2) (layer "F.Cu") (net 3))
 (segment (start 42.7 76.1) (end 41.7865 75.1865) (width 0.3) (layer "F.Cu") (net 3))
 (segment (start 134.1 78.15) (end 133.9 78.35) (width 0.3) (layer "F.Cu") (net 3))
 (segment (start 44.05 78.35) (end 42.7 77) (width 0.3) (layer "F.Cu") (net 3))
 (segment (start 41.3 75.2032) (end 41.8032 75.2032) (width 0.2) (layer "F.Cu") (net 3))
 (segment (start 135.5968 75.4032) (end 135.7968 75.2032) (width 0.2) (layer "F.Cu") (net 3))
 (segment (start 135.5968 75.4032) (end 134.1 76.9) (width 0.25) (layer "F.Cu") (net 3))
 (segment (start 134.1 76.9) (end 134.1 77.05) (width 0.25) (layer "F.Cu") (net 3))
 (segment (start 42.7 77) (end 42.7 76.1) (width 0.3) (layer "F.Cu") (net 3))
 (via (at 134.1 77.05) (size 0.6) (drill 0.3) (layers "F.Cu" "B.Cu") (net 3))
 (via (at 134.1 78.15) (size 0.6) (drill 0.3) (layers "F.Cu" "B.Cu") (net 3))
 (segment (start 134.1 77.05) (end 134.1 78.15) (width 0.25) (layer "B.Cu") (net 3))
 (segment (start 43.7 75.2032) (end 44.1968 75.2032) (width 0.2) (layer "F.Cu") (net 6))
 (segment (start 44.2 75.2) (end 44.4 75.4) (width 0.2) (layer "F.Cu") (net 6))
 (segment (start 138.3634 75.2032) (end 138.2968 75.2032) (width 0.3) (layer "F.Cu") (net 6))
 (segment (start 137.6 77) (end 137 77.6) (width 0.3) (layer "F.Cu") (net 6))
 (segment (start 44.85 77.6) (end 44.4 77.15) (width 0.3) (layer "F.Cu") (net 6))
 (segment (start 44.4 77.15) (end 44.4 75.4) (width 0.3) (layer "F.Cu") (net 6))
 (segment (start 138.3634 75.2032) (end 138.7 75.2032) (width 0.2) (layer "F.Cu") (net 6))
 (segment (start 138.2968 75.2032) (end 137.6 75.9) (width 0.3) (layer "F.Cu") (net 6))
 (segment (start 137.6 75.9) (end 137.6 77) (width 0.3) (layer "F.Cu") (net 6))
 (segment (start 137 77.6) (end 44.85 77.6) (width 0.3) (layer "F.Cu") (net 6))
 (segment (start 44.1968 75.2032) (end 44.2 75.2) (width 0.2) (layer "F.Cu") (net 6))
 (segment (start 134.9 72) (end 134.9 73.959704) (width 0.3) (layer "F.Cu") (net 2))
 (segment (start 41.9032 74.7968) (end 41.3 74.7968) (width 0.2) (layer "F.Cu") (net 2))
 (segment (start 134.7 71.8) (end 134.9 72) (width 0.3) (layer "F.Cu") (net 2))
 (segment (start 42.4 74) (end 44.6 71.8) (width 0.3) (layer "F.Cu") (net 2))
 (segment (start 135.737096 74.7968) (end 135.370148 74.429852) (width 0.2) (layer "F.Cu") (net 2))
 (segment (start 42.4 74.3) (end 42.4 74) (width 0.3) (layer "F.Cu") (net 2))
 (segment (start 44.6 71.8) (end 134.7 71.8) (width 0.3) (layer "F.Cu") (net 2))
 (segment (start 42.4 74.3) (end 41.9032 74.7968) (width 0.2) (layer "F.Cu") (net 2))
 (segment (start 134.9 73.959704) (end 135.370148 74.429852) (width 0.3) (layer "F.Cu") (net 2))
 (segment (start 136.3 74.7968) (end 135.737096 74.7968) (width 0.2) (layer "F.Cu") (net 2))
 (segment (start 47.4 75.1) (end 49 75.1) (width 0.3) (layer "F.Cu") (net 12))
 (segment (start 45.4 76.45) (end 46.05 76.45) (width 0.3) (layer "F.Cu") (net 12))
 (segment (start 46.05 76.45) (end 47.4 75.1) (width 0.3) (layer "F.Cu") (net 12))
 (segment (start 50.75 73.35) (end 52.45 73.35) (width 0.3) (layer "F.Cu") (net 12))
 (segment (start 49 75.1) (end 50.75 73.35) (width 0.3) (layer "F.Cu") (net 12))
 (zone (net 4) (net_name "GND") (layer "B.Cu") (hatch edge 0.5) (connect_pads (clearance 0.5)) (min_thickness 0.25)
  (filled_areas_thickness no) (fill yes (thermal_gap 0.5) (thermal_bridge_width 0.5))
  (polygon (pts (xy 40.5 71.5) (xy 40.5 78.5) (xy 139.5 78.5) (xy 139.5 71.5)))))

